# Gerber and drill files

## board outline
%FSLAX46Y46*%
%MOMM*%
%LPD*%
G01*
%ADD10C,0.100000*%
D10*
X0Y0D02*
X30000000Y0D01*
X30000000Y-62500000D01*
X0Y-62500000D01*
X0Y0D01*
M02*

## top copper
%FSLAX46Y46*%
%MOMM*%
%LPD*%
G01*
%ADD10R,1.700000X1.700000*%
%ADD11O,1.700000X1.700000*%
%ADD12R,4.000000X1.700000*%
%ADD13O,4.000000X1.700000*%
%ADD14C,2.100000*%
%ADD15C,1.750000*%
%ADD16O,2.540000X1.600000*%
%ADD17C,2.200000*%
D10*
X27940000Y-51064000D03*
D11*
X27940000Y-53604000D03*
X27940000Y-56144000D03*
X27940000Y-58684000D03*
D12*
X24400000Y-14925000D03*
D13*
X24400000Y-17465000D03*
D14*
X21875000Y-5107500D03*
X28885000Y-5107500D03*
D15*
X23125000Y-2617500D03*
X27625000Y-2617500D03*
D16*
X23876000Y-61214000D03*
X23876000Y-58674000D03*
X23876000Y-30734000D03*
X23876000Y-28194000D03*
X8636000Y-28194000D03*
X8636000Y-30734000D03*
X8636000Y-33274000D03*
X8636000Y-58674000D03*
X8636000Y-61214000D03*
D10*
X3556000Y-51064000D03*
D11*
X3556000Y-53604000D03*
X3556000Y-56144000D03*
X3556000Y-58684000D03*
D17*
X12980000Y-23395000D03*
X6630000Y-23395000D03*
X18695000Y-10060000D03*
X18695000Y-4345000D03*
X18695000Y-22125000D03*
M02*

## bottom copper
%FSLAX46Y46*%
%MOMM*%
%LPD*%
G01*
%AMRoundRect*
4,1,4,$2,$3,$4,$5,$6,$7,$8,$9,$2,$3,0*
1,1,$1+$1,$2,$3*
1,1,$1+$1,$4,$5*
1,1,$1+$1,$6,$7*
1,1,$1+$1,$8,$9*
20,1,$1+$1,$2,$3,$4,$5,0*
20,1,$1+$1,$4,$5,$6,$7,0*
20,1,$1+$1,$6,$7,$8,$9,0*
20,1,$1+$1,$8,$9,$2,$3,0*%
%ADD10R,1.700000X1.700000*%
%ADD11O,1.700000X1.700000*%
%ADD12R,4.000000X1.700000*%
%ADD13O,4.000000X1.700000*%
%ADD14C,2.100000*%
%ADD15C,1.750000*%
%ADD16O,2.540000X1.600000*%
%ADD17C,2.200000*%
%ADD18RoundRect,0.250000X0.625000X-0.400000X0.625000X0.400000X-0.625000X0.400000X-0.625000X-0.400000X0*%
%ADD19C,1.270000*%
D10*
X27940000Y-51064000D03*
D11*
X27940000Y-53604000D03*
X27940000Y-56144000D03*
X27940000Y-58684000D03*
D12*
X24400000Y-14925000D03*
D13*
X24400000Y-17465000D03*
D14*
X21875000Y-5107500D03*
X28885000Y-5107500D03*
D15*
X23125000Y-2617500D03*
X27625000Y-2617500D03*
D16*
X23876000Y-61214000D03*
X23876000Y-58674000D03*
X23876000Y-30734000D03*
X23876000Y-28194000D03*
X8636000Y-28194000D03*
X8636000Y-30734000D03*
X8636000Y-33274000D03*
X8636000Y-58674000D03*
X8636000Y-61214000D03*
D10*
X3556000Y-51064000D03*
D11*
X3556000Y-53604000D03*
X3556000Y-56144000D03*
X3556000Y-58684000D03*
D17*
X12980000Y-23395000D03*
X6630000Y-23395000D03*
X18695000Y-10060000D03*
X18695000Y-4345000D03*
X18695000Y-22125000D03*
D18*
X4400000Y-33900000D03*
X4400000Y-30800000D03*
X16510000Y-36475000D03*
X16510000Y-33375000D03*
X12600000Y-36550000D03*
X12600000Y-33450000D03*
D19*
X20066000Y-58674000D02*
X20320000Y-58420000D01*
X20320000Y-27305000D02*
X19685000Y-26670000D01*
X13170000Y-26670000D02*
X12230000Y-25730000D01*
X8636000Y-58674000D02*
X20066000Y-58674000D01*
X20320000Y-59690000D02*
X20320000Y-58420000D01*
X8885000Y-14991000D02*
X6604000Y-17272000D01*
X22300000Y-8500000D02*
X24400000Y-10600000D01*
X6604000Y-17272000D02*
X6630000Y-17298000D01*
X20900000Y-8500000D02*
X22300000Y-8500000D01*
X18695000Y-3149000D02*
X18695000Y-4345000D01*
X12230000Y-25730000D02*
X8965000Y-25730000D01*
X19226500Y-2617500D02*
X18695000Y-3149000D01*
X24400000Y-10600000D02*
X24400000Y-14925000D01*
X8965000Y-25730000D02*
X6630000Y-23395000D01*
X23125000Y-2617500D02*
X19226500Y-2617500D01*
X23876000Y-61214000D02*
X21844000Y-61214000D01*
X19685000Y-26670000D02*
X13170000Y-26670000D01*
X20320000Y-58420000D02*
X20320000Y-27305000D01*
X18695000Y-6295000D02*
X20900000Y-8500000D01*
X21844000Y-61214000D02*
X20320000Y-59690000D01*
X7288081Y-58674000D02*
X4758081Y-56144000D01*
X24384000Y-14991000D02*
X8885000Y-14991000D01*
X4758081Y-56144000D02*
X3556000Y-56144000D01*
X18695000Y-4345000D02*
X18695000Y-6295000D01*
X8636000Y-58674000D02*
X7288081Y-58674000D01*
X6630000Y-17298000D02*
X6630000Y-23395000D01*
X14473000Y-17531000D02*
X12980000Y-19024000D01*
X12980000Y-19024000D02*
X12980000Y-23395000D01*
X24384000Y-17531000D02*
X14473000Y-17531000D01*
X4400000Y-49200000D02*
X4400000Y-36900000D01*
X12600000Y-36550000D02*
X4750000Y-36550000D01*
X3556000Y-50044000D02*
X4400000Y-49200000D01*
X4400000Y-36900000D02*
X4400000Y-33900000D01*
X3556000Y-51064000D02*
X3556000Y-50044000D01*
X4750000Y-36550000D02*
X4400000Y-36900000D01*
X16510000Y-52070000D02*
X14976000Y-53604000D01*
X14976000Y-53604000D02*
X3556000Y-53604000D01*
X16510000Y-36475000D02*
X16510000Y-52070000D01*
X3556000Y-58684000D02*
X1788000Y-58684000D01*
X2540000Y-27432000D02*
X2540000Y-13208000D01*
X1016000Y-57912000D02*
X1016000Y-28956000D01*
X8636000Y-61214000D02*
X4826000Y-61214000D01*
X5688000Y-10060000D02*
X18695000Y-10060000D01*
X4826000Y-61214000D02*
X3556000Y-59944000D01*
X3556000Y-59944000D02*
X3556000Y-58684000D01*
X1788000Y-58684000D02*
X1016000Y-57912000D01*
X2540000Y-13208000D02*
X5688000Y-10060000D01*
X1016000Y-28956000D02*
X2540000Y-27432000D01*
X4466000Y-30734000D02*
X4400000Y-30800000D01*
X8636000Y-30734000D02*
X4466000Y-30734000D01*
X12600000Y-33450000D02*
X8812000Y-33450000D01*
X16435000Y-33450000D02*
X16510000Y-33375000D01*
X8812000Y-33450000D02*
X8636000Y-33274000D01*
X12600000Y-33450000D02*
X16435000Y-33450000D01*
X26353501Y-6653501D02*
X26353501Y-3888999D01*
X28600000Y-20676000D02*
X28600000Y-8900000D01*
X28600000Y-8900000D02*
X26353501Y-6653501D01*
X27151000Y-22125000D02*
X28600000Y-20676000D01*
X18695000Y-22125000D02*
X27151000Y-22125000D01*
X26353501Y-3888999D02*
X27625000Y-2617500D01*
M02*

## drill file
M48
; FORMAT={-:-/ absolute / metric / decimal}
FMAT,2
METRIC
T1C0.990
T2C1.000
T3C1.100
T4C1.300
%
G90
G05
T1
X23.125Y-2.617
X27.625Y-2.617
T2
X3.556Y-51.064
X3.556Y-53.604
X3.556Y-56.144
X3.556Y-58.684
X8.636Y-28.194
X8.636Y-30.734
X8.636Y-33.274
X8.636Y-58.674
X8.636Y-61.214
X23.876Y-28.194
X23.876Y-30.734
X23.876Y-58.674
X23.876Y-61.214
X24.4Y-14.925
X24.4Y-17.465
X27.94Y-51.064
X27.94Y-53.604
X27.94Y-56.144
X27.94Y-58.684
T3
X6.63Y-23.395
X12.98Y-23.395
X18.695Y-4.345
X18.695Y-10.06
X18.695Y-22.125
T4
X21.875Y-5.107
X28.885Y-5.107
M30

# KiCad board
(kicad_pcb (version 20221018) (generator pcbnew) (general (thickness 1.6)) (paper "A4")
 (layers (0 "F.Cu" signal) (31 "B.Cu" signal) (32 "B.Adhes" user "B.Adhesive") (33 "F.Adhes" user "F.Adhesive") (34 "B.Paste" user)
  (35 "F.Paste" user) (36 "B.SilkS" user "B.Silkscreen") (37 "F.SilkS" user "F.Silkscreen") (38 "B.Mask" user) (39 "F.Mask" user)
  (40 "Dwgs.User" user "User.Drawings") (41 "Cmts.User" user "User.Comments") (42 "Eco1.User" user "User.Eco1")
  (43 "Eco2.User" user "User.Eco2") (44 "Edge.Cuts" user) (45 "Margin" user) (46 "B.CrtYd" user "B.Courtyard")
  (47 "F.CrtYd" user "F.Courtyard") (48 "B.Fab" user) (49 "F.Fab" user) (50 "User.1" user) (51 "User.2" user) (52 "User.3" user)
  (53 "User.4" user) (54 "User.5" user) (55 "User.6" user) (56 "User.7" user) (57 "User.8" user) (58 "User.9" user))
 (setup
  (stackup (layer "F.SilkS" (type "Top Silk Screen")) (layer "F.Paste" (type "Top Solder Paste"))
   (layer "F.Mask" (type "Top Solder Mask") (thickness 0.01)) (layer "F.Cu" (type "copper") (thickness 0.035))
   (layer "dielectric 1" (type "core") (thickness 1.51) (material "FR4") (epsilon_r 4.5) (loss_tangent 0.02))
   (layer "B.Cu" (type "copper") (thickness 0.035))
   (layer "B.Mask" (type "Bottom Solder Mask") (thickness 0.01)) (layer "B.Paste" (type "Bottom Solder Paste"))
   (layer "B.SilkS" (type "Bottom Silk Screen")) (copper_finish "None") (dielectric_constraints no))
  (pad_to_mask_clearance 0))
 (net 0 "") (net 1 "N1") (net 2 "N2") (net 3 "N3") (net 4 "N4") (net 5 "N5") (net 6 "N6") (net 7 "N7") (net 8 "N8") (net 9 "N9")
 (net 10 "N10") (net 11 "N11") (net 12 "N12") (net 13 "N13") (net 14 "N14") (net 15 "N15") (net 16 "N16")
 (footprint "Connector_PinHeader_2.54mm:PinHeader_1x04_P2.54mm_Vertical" (layer "F.Cu") (at 27.94 51.064)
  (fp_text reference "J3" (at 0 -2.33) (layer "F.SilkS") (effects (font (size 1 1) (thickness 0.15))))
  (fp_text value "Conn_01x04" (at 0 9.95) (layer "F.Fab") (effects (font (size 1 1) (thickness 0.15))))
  (pad "1" thru_hole rect (at 0 0) (size 1.7 1.7) (drill 1) (layers "*.Cu" "*.Mask") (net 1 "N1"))
  (pad "2" thru_hole oval (at 0 2.54) (size 1.7 1.7) (drill 1) (layers "*.Cu" "*.Mask") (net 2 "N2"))
  (pad "3" thru_hole oval (at 0 5.08) (size 1.7 1.7) (drill 1) (layers "*.Cu" "*.Mask") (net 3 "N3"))
  (pad "4" thru_hole oval (at 0 7.62) (size 1.7 1.7) (drill 1) (layers "*.Cu" "*.Mask") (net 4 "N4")))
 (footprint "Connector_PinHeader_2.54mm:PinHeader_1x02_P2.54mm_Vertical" (layer "F.Cu") (at 24.4 14.925)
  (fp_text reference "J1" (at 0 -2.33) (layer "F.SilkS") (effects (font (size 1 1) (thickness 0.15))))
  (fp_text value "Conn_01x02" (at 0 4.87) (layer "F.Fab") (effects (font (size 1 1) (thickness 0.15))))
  (pad "1" thru_hole rect (at 0 0) (size 4 1.7) (drill 1) (layers "*.Cu" "*.Mask") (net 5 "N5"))
  (pad "2" thru_hole oval (at 0 2.54) (size 4 1.7) (drill 1) (layers "*.Cu" "*.Mask") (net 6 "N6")))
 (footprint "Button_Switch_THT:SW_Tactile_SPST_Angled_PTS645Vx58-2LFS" (layer "F.Cu") (at 23.125 2.6175)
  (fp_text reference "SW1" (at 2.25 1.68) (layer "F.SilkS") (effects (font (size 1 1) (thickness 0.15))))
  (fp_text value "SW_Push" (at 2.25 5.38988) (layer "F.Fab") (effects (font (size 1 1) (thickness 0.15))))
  (pad "" thru_hole circle (at -1.25 2.49) (size 2.1 2.1) (drill 1.3) (layers "*.Cu" "*.Mask"))
  (pad "" thru_hole circle (at 5.76 2.49) (size 2.1 2.1) (drill 1.3) (layers "*.Cu" "*.Mask"))
  (pad "1" thru_hole circle (at 0 0) (size 1.75 1.75) (drill 0.99) (layers "*.Cu" "*.Mask") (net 5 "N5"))
  (pad "2" thru_hole circle (at 4.5 0) (size 1.75 1.75) (drill 0.99) (layers "*.Cu" "*.Mask") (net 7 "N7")))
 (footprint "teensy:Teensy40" (layer "F.Cu") (at 16.256 44.704 90)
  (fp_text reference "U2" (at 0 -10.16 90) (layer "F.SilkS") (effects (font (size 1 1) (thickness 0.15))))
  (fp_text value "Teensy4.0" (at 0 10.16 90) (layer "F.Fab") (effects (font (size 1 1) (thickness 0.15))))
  (pad "1" thru_hole oval (at -16.51 7.62 90) (size 1.6 2.54) (drill 1) (layers "*.Cu" "*.Mask") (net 5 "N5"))
  (pad "2" thru_hole oval (at -13.97 7.62 90) (size 1.6 2.54) (drill 1) (layers "*.Cu" "*.Mask") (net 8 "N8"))
  (pad "13" thru_hole oval (at 13.97 7.62 90) (size 1.6 2.54) (drill 1) (layers "*.Cu" "*.Mask") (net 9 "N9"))
  (pad "14" thru_hole oval (at 16.51 7.62 90) (size 1.6 2.54) (drill 1) (layers "*.Cu" "*.Mask") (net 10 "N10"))
  (pad "20" thru_hole oval (at 16.51 -7.62 90) (size 1.6 2.54) (drill 1) (layers "*.Cu" "*.Mask") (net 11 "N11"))
  (pad "21" thru_hole oval (at 13.97 -7.62 90) (size 1.6 2.54) (drill 1) (layers "*.Cu" "*.Mask") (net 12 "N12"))
  (pad "22" thru_hole oval (at 11.43 -7.62 90) (size 1.6 2.54) (drill 1) (layers "*.Cu" "*.Mask") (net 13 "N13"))
  (pad "32" thru_hole oval (at -13.97 -7.62 90) (size 1.6 2.54) (drill 1) (layers "*.Cu" "*.Mask") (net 5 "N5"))
  (pad "33" thru_hole oval (at -16.51 -7.62 90) (size 1.6 2.54) (drill 1) (layers "*.Cu" "*.Mask") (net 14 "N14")))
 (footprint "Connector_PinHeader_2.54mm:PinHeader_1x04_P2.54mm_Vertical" (layer "F.Cu") (at 3.556 51.064)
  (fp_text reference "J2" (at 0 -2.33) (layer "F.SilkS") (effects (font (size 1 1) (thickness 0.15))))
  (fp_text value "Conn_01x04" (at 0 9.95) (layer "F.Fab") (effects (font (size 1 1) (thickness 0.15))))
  (pad "1" thru_hole rect (at 0 0) (size 1.7 1.7) (drill 1) (layers "*.Cu" "*.Mask") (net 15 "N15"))
  (pad "2" thru_hole oval (at 0 2.54) (size 1.7 1.7) (drill 1) (layers "*.Cu" "*.Mask") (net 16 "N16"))
  (pad "3" thru_hole oval (at 0 5.08) (size 1.7 1.7) (drill 1) (layers "*.Cu" "*.Mask") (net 5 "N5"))
  (pad "4" thru_hole oval (at 0 7.62) (size 1.7 1.7) (drill 1) (layers "*.Cu" "*.Mask") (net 14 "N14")))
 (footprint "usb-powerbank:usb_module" (layer "F.Cu") (at 0.045 0)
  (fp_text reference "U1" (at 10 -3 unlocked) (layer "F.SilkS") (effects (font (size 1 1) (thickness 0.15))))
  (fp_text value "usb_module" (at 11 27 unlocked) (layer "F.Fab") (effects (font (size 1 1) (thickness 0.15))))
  (pad "1" thru_hole circle (at 12.935 23.395) (size 2.2 2.2) (drill 1.1) (layers "*.Cu" "*.Mask") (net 6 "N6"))
  (pad "2" thru_hole circle (at 6.585 23.395) (size 2.2 2.2) (drill 1.1) (layers "*.Cu" "*.Mask") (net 5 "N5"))
  (pad "3" thru_hole circle (at 18.65 10.06) (size 2.2 2.2) (drill 1.1) (layers "*.Cu" "*.Mask") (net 14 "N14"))
  (pad "4" thru_hole circle (at 18.65 4.345) (size 2.2 2.2) (drill 1.1) (layers "*.Cu" "*.Mask") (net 5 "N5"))
  (pad "5" thru_hole circle (at 18.65 22.125) (size 2.2 2.2) (drill 1.1) (layers "*.Cu" "*.Mask") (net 7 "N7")))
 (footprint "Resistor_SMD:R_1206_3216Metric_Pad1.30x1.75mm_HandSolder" (layer "B.Cu") (at 4.4 32.35 90)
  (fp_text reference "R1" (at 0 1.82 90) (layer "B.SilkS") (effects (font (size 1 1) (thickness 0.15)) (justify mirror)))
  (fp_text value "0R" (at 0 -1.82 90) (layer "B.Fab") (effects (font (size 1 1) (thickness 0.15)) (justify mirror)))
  (pad "1" smd roundrect (at -1.55 0 90) (size 1.3 1.75) (layers "B.Cu" "B.Paste" "B.Mask") (roundrect_rratio 0.1923076923) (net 15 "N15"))
  (pad "2" smd roundrect (at 1.55 0 90) (size 1.3 1.75) (layers "B.Cu" "B.Paste" "B.Mask") (roundrect_rratio 0.1923076923) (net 12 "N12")))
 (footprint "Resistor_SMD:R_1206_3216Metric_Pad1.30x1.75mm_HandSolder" (layer "B.Cu") (at 16.51 34.925 90)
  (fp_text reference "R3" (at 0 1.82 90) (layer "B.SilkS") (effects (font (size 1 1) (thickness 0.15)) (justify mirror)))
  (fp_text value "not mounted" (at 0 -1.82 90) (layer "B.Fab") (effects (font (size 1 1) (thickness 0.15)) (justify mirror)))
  (pad "1" smd roundrect (at -1.55 0 90) (size 1.3 1.75) (layers "B.Cu" "B.Paste" "B.Mask") (roundrect_rratio 0.1923076923) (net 16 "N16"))
  (pad "2" smd roundrect (at 1.55 0 90) (size 1.3 1.75) (layers "B.Cu" "B.Paste" "B.Mask") (roundrect_rratio 0.1923076923) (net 13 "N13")))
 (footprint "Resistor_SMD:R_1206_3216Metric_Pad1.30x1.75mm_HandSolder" (layer "B.Cu") (at 12.6 35 90)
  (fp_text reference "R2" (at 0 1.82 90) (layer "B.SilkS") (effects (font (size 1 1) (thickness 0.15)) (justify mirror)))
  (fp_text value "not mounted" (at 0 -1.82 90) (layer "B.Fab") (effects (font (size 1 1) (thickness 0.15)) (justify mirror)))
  (pad "1" smd roundrect (at -1.55 0 90) (size 1.3 1.75) (layers "B.Cu" "B.Paste" "B.Mask") (roundrect_rratio 0.1923076923) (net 15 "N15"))
  (pad "2" smd roundrect (at 1.55 0 90) (size 1.3 1.75) (layers "B.Cu" "B.Paste" "B.Mask") (roundrect_rratio 0.1923076923) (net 13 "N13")))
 (gr_rect (start 0 0) (end 30 62.5) (stroke (width 0.1) (type solid)) (fill none) (layer "Edge.Cuts"))
 (segment (start 20.066 58.674) (end 20.32 58.42) (width 1.27) (layer "B.Cu") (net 5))
 (segment (start 20.32 27.305) (end 19.685 26.67) (width 1.27) (layer "B.Cu") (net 5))
 (segment (start 13.17 26.67) (end 12.23 25.73) (width 1.27) (layer "B.Cu") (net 5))
 (segment (start 8.636 58.674) (end 20.066 58.674) (width 1.27) (layer "B.Cu") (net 5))
 (segment (start 20.32 59.69) (end 20.32 58.42) (width 1.27) (layer "B.Cu") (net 5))
 (segment (start 8.885 14.991) (end 6.604 17.272) (width 1.27) (layer "B.Cu") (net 5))
 (segment (start 22.3 8.5) (end 24.4 10.6) (width 1.27) (layer "B.Cu") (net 5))
 (segment (start 6.604 17.272) (end 6.63 17.298) (width 1.27) (layer "B.Cu") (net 5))
 (segment (start 20.9 8.5) (end 22.3 8.5) (width 1.27) (layer "B.Cu") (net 5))
 (segment (start 18.695 3.149) (end 18.695 4.345) (width 1.27) (layer "B.Cu") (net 5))
 (segment (start 12.23 25.73) (end 8.965 25.73) (width 1.27) (layer "B.Cu") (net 5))
 (segment (start 19.2265 2.6175) (end 18.695 3.149) (width 1.27) (layer "B.Cu") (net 5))
 (segment (start 24.4 10.6) (end 24.4 14.925) (width 1.27) (layer "B.Cu") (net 5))
 (segment (start 8.965 25.73) (end 6.63 23.395) (width 1.27) (layer "B.Cu") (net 5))
 (segment (start 23.125 2.6175) (end 19.2265 2.6175) (width 1.27) (layer "B.Cu") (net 5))
 (segment (start 23.876 61.214) (end 21.844 61.214) (width 1.27) (layer "B.Cu") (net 5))
 (segment (start 19.685 26.67) (end 13.17 26.67) (width 1.27) (layer "B.Cu") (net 5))
 (segment (start 20.32 58.42) (end 20.32 27.305) (width 1.27) (layer "B.Cu") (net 5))
 (segment (start 18.695 6.295) (end 20.9 8.5) (width 1.27) (layer "B.Cu") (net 5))
 (segment (start 21.844 61.214) (end 20.32 59.69) (width 1.27) (layer "B.Cu") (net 5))
 (segment (start 7.288081 58.674) (end 4.758081 56.144) (width 1.27) (layer "B.Cu") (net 5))
 (segment (start 24.384 14.991) (end 8.885 14.991) (width 1.27) (layer "B.Cu") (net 5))
 (segment (start 4.758081 56.144) (end 3.556 56.144) (width 1.27) (layer "B.Cu") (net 5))
 (segment (start 18.695 4.345) (end 18.695 6.295) (width 1.27) (layer "B.Cu") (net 5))
 (segment (start 8.636 58.674) (end 7.288081 58.674) (width 1.27) (layer "B.Cu") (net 5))
 (segment (start 6.63 17.298) (end 6.63 23.395) (width 1.27) (layer "B.Cu") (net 5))
 (segment (start 14.473 17.531) (end 12.98 19.024) (width 1.27) (layer "B.Cu") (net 6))
 (segment (start 12.98 19.024) (end 12.98 23.395) (width 1.27) (layer "B.Cu") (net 6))
 (segment (start 24.384 17.531) (end 14.473 17.531) (width 1.27) (layer "B.Cu") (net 6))
 (segment (start 4.4 49.2) (end 4.4 36.9) (width 1.27) (layer "B.Cu") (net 15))
 (segment (start 12.6 36.55) (end 4.75 36.55) (width 1.27) (layer "B.Cu") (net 15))
 (segment (start 3.556 50.044) (end 4.4 49.2) (width 1.27) (layer "B.Cu") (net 15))
 (segment (start 4.4 36.9) (end 4.4 33.9) (width 1.27) (layer "B.Cu") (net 15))
 (segment (start 3.556 51.064) (end 3.556 50.044) (width 1.27) (layer "B.Cu") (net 15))
 (segment (start 4.75 36.55) (end 4.4 36.9) (width 1.27) (layer "B.Cu") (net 15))
 (segment (start 16.51 52.07) (end 14.976 53.604) (width 1.27) (layer "B.Cu") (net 16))
 (segment (start 14.976 53.604) (end 3.556 53.604) (width 1.27) (layer "B.Cu") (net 16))
 (segment (start 16.51 36.475) (end 16.51 52.07) (width 1.27) (layer "B.Cu") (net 16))
 (segment (start 3.556 58.684) (end 1.788 58.684) (width 1.27) (layer "B.Cu") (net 14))
 (segment (start 2.54 27.432) (end 2.54 13.208) (width 1.27) (layer "B.Cu") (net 14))
 (segment (start 1.016 57.912) (end 1.016 28.956) (width 1.27) (layer "B.Cu") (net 14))
 (segment (start 8.636 61.214) (end 4.826 61.214) (width 1.27) (layer "B.Cu") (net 14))
 (segment (start 5.688 10.06) (end 18.695 10.06) (width 1.27) (layer "B.Cu") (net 14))
 (segment (start 4.826 61.214) (end 3.556 59.944) (width 1.27) (layer "B.Cu") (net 14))
 (segment (start 3.556 59.944) (end 3.556 58.684) (width 1.27) (layer "B.Cu") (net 14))
 (segment (start 1.788 58.684) (end 1.016 57.912) (width 1.27) (layer "B.Cu") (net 14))
 (segment (start 2.54 13.208) (end 5.688 10.06) (width 1.27) (layer "B.Cu") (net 14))
 (segment (start 1.016 28.956) (end 2.54 27.432) (width 1.27) (layer "B.Cu") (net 14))
 (segment (start 4.466 30.734) (end 4.4 30.8) (width 1.27) (layer "B.Cu") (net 12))
 (segment (start 8.636 30.734) (end 4.466 30.734) (width 1.27) (layer "B.Cu") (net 12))
 (segment (start 12.6 33.45) (end 8.812 33.45) (width 1.27) (layer "B.Cu") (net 13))
 (segment (start 16.435 33.45) (end 16.51 33.375) (width 1.27) (layer "B.Cu") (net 13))
 (segment (start 8.812 33.45) (end 8.636 33.274) (width 1.27) (layer "B.Cu") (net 13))
 (segment (start 12.6 33.45) (end 16.435 33.45) (width 1.27) (layer "B.Cu") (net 13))
 (segment (start 26.353501 6.653501) (end 26.353501 3.888999) (width 1.27) (layer "B.Cu") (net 7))
 (segment (start 28.6 20.676) (end 28.6 8.9) (width 1.27) (layer "B.Cu") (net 7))
 (segment (start 28.6 8.9) (end 26.353501 6.653501) (width 1.27) (layer "B.Cu") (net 7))
 (segment (start 27.151 22.125) (end 28.6 20.676) (width 1.27) (layer "B.Cu") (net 7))
 (segment (start 18.695 22.125) (end 27.151 22.125) (width 1.27) (layer "B.Cu") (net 7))
 (segment (start 26.353501 3.888999) (end 27.625 2.6175) (width 1.27) (layer "B.Cu") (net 7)))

